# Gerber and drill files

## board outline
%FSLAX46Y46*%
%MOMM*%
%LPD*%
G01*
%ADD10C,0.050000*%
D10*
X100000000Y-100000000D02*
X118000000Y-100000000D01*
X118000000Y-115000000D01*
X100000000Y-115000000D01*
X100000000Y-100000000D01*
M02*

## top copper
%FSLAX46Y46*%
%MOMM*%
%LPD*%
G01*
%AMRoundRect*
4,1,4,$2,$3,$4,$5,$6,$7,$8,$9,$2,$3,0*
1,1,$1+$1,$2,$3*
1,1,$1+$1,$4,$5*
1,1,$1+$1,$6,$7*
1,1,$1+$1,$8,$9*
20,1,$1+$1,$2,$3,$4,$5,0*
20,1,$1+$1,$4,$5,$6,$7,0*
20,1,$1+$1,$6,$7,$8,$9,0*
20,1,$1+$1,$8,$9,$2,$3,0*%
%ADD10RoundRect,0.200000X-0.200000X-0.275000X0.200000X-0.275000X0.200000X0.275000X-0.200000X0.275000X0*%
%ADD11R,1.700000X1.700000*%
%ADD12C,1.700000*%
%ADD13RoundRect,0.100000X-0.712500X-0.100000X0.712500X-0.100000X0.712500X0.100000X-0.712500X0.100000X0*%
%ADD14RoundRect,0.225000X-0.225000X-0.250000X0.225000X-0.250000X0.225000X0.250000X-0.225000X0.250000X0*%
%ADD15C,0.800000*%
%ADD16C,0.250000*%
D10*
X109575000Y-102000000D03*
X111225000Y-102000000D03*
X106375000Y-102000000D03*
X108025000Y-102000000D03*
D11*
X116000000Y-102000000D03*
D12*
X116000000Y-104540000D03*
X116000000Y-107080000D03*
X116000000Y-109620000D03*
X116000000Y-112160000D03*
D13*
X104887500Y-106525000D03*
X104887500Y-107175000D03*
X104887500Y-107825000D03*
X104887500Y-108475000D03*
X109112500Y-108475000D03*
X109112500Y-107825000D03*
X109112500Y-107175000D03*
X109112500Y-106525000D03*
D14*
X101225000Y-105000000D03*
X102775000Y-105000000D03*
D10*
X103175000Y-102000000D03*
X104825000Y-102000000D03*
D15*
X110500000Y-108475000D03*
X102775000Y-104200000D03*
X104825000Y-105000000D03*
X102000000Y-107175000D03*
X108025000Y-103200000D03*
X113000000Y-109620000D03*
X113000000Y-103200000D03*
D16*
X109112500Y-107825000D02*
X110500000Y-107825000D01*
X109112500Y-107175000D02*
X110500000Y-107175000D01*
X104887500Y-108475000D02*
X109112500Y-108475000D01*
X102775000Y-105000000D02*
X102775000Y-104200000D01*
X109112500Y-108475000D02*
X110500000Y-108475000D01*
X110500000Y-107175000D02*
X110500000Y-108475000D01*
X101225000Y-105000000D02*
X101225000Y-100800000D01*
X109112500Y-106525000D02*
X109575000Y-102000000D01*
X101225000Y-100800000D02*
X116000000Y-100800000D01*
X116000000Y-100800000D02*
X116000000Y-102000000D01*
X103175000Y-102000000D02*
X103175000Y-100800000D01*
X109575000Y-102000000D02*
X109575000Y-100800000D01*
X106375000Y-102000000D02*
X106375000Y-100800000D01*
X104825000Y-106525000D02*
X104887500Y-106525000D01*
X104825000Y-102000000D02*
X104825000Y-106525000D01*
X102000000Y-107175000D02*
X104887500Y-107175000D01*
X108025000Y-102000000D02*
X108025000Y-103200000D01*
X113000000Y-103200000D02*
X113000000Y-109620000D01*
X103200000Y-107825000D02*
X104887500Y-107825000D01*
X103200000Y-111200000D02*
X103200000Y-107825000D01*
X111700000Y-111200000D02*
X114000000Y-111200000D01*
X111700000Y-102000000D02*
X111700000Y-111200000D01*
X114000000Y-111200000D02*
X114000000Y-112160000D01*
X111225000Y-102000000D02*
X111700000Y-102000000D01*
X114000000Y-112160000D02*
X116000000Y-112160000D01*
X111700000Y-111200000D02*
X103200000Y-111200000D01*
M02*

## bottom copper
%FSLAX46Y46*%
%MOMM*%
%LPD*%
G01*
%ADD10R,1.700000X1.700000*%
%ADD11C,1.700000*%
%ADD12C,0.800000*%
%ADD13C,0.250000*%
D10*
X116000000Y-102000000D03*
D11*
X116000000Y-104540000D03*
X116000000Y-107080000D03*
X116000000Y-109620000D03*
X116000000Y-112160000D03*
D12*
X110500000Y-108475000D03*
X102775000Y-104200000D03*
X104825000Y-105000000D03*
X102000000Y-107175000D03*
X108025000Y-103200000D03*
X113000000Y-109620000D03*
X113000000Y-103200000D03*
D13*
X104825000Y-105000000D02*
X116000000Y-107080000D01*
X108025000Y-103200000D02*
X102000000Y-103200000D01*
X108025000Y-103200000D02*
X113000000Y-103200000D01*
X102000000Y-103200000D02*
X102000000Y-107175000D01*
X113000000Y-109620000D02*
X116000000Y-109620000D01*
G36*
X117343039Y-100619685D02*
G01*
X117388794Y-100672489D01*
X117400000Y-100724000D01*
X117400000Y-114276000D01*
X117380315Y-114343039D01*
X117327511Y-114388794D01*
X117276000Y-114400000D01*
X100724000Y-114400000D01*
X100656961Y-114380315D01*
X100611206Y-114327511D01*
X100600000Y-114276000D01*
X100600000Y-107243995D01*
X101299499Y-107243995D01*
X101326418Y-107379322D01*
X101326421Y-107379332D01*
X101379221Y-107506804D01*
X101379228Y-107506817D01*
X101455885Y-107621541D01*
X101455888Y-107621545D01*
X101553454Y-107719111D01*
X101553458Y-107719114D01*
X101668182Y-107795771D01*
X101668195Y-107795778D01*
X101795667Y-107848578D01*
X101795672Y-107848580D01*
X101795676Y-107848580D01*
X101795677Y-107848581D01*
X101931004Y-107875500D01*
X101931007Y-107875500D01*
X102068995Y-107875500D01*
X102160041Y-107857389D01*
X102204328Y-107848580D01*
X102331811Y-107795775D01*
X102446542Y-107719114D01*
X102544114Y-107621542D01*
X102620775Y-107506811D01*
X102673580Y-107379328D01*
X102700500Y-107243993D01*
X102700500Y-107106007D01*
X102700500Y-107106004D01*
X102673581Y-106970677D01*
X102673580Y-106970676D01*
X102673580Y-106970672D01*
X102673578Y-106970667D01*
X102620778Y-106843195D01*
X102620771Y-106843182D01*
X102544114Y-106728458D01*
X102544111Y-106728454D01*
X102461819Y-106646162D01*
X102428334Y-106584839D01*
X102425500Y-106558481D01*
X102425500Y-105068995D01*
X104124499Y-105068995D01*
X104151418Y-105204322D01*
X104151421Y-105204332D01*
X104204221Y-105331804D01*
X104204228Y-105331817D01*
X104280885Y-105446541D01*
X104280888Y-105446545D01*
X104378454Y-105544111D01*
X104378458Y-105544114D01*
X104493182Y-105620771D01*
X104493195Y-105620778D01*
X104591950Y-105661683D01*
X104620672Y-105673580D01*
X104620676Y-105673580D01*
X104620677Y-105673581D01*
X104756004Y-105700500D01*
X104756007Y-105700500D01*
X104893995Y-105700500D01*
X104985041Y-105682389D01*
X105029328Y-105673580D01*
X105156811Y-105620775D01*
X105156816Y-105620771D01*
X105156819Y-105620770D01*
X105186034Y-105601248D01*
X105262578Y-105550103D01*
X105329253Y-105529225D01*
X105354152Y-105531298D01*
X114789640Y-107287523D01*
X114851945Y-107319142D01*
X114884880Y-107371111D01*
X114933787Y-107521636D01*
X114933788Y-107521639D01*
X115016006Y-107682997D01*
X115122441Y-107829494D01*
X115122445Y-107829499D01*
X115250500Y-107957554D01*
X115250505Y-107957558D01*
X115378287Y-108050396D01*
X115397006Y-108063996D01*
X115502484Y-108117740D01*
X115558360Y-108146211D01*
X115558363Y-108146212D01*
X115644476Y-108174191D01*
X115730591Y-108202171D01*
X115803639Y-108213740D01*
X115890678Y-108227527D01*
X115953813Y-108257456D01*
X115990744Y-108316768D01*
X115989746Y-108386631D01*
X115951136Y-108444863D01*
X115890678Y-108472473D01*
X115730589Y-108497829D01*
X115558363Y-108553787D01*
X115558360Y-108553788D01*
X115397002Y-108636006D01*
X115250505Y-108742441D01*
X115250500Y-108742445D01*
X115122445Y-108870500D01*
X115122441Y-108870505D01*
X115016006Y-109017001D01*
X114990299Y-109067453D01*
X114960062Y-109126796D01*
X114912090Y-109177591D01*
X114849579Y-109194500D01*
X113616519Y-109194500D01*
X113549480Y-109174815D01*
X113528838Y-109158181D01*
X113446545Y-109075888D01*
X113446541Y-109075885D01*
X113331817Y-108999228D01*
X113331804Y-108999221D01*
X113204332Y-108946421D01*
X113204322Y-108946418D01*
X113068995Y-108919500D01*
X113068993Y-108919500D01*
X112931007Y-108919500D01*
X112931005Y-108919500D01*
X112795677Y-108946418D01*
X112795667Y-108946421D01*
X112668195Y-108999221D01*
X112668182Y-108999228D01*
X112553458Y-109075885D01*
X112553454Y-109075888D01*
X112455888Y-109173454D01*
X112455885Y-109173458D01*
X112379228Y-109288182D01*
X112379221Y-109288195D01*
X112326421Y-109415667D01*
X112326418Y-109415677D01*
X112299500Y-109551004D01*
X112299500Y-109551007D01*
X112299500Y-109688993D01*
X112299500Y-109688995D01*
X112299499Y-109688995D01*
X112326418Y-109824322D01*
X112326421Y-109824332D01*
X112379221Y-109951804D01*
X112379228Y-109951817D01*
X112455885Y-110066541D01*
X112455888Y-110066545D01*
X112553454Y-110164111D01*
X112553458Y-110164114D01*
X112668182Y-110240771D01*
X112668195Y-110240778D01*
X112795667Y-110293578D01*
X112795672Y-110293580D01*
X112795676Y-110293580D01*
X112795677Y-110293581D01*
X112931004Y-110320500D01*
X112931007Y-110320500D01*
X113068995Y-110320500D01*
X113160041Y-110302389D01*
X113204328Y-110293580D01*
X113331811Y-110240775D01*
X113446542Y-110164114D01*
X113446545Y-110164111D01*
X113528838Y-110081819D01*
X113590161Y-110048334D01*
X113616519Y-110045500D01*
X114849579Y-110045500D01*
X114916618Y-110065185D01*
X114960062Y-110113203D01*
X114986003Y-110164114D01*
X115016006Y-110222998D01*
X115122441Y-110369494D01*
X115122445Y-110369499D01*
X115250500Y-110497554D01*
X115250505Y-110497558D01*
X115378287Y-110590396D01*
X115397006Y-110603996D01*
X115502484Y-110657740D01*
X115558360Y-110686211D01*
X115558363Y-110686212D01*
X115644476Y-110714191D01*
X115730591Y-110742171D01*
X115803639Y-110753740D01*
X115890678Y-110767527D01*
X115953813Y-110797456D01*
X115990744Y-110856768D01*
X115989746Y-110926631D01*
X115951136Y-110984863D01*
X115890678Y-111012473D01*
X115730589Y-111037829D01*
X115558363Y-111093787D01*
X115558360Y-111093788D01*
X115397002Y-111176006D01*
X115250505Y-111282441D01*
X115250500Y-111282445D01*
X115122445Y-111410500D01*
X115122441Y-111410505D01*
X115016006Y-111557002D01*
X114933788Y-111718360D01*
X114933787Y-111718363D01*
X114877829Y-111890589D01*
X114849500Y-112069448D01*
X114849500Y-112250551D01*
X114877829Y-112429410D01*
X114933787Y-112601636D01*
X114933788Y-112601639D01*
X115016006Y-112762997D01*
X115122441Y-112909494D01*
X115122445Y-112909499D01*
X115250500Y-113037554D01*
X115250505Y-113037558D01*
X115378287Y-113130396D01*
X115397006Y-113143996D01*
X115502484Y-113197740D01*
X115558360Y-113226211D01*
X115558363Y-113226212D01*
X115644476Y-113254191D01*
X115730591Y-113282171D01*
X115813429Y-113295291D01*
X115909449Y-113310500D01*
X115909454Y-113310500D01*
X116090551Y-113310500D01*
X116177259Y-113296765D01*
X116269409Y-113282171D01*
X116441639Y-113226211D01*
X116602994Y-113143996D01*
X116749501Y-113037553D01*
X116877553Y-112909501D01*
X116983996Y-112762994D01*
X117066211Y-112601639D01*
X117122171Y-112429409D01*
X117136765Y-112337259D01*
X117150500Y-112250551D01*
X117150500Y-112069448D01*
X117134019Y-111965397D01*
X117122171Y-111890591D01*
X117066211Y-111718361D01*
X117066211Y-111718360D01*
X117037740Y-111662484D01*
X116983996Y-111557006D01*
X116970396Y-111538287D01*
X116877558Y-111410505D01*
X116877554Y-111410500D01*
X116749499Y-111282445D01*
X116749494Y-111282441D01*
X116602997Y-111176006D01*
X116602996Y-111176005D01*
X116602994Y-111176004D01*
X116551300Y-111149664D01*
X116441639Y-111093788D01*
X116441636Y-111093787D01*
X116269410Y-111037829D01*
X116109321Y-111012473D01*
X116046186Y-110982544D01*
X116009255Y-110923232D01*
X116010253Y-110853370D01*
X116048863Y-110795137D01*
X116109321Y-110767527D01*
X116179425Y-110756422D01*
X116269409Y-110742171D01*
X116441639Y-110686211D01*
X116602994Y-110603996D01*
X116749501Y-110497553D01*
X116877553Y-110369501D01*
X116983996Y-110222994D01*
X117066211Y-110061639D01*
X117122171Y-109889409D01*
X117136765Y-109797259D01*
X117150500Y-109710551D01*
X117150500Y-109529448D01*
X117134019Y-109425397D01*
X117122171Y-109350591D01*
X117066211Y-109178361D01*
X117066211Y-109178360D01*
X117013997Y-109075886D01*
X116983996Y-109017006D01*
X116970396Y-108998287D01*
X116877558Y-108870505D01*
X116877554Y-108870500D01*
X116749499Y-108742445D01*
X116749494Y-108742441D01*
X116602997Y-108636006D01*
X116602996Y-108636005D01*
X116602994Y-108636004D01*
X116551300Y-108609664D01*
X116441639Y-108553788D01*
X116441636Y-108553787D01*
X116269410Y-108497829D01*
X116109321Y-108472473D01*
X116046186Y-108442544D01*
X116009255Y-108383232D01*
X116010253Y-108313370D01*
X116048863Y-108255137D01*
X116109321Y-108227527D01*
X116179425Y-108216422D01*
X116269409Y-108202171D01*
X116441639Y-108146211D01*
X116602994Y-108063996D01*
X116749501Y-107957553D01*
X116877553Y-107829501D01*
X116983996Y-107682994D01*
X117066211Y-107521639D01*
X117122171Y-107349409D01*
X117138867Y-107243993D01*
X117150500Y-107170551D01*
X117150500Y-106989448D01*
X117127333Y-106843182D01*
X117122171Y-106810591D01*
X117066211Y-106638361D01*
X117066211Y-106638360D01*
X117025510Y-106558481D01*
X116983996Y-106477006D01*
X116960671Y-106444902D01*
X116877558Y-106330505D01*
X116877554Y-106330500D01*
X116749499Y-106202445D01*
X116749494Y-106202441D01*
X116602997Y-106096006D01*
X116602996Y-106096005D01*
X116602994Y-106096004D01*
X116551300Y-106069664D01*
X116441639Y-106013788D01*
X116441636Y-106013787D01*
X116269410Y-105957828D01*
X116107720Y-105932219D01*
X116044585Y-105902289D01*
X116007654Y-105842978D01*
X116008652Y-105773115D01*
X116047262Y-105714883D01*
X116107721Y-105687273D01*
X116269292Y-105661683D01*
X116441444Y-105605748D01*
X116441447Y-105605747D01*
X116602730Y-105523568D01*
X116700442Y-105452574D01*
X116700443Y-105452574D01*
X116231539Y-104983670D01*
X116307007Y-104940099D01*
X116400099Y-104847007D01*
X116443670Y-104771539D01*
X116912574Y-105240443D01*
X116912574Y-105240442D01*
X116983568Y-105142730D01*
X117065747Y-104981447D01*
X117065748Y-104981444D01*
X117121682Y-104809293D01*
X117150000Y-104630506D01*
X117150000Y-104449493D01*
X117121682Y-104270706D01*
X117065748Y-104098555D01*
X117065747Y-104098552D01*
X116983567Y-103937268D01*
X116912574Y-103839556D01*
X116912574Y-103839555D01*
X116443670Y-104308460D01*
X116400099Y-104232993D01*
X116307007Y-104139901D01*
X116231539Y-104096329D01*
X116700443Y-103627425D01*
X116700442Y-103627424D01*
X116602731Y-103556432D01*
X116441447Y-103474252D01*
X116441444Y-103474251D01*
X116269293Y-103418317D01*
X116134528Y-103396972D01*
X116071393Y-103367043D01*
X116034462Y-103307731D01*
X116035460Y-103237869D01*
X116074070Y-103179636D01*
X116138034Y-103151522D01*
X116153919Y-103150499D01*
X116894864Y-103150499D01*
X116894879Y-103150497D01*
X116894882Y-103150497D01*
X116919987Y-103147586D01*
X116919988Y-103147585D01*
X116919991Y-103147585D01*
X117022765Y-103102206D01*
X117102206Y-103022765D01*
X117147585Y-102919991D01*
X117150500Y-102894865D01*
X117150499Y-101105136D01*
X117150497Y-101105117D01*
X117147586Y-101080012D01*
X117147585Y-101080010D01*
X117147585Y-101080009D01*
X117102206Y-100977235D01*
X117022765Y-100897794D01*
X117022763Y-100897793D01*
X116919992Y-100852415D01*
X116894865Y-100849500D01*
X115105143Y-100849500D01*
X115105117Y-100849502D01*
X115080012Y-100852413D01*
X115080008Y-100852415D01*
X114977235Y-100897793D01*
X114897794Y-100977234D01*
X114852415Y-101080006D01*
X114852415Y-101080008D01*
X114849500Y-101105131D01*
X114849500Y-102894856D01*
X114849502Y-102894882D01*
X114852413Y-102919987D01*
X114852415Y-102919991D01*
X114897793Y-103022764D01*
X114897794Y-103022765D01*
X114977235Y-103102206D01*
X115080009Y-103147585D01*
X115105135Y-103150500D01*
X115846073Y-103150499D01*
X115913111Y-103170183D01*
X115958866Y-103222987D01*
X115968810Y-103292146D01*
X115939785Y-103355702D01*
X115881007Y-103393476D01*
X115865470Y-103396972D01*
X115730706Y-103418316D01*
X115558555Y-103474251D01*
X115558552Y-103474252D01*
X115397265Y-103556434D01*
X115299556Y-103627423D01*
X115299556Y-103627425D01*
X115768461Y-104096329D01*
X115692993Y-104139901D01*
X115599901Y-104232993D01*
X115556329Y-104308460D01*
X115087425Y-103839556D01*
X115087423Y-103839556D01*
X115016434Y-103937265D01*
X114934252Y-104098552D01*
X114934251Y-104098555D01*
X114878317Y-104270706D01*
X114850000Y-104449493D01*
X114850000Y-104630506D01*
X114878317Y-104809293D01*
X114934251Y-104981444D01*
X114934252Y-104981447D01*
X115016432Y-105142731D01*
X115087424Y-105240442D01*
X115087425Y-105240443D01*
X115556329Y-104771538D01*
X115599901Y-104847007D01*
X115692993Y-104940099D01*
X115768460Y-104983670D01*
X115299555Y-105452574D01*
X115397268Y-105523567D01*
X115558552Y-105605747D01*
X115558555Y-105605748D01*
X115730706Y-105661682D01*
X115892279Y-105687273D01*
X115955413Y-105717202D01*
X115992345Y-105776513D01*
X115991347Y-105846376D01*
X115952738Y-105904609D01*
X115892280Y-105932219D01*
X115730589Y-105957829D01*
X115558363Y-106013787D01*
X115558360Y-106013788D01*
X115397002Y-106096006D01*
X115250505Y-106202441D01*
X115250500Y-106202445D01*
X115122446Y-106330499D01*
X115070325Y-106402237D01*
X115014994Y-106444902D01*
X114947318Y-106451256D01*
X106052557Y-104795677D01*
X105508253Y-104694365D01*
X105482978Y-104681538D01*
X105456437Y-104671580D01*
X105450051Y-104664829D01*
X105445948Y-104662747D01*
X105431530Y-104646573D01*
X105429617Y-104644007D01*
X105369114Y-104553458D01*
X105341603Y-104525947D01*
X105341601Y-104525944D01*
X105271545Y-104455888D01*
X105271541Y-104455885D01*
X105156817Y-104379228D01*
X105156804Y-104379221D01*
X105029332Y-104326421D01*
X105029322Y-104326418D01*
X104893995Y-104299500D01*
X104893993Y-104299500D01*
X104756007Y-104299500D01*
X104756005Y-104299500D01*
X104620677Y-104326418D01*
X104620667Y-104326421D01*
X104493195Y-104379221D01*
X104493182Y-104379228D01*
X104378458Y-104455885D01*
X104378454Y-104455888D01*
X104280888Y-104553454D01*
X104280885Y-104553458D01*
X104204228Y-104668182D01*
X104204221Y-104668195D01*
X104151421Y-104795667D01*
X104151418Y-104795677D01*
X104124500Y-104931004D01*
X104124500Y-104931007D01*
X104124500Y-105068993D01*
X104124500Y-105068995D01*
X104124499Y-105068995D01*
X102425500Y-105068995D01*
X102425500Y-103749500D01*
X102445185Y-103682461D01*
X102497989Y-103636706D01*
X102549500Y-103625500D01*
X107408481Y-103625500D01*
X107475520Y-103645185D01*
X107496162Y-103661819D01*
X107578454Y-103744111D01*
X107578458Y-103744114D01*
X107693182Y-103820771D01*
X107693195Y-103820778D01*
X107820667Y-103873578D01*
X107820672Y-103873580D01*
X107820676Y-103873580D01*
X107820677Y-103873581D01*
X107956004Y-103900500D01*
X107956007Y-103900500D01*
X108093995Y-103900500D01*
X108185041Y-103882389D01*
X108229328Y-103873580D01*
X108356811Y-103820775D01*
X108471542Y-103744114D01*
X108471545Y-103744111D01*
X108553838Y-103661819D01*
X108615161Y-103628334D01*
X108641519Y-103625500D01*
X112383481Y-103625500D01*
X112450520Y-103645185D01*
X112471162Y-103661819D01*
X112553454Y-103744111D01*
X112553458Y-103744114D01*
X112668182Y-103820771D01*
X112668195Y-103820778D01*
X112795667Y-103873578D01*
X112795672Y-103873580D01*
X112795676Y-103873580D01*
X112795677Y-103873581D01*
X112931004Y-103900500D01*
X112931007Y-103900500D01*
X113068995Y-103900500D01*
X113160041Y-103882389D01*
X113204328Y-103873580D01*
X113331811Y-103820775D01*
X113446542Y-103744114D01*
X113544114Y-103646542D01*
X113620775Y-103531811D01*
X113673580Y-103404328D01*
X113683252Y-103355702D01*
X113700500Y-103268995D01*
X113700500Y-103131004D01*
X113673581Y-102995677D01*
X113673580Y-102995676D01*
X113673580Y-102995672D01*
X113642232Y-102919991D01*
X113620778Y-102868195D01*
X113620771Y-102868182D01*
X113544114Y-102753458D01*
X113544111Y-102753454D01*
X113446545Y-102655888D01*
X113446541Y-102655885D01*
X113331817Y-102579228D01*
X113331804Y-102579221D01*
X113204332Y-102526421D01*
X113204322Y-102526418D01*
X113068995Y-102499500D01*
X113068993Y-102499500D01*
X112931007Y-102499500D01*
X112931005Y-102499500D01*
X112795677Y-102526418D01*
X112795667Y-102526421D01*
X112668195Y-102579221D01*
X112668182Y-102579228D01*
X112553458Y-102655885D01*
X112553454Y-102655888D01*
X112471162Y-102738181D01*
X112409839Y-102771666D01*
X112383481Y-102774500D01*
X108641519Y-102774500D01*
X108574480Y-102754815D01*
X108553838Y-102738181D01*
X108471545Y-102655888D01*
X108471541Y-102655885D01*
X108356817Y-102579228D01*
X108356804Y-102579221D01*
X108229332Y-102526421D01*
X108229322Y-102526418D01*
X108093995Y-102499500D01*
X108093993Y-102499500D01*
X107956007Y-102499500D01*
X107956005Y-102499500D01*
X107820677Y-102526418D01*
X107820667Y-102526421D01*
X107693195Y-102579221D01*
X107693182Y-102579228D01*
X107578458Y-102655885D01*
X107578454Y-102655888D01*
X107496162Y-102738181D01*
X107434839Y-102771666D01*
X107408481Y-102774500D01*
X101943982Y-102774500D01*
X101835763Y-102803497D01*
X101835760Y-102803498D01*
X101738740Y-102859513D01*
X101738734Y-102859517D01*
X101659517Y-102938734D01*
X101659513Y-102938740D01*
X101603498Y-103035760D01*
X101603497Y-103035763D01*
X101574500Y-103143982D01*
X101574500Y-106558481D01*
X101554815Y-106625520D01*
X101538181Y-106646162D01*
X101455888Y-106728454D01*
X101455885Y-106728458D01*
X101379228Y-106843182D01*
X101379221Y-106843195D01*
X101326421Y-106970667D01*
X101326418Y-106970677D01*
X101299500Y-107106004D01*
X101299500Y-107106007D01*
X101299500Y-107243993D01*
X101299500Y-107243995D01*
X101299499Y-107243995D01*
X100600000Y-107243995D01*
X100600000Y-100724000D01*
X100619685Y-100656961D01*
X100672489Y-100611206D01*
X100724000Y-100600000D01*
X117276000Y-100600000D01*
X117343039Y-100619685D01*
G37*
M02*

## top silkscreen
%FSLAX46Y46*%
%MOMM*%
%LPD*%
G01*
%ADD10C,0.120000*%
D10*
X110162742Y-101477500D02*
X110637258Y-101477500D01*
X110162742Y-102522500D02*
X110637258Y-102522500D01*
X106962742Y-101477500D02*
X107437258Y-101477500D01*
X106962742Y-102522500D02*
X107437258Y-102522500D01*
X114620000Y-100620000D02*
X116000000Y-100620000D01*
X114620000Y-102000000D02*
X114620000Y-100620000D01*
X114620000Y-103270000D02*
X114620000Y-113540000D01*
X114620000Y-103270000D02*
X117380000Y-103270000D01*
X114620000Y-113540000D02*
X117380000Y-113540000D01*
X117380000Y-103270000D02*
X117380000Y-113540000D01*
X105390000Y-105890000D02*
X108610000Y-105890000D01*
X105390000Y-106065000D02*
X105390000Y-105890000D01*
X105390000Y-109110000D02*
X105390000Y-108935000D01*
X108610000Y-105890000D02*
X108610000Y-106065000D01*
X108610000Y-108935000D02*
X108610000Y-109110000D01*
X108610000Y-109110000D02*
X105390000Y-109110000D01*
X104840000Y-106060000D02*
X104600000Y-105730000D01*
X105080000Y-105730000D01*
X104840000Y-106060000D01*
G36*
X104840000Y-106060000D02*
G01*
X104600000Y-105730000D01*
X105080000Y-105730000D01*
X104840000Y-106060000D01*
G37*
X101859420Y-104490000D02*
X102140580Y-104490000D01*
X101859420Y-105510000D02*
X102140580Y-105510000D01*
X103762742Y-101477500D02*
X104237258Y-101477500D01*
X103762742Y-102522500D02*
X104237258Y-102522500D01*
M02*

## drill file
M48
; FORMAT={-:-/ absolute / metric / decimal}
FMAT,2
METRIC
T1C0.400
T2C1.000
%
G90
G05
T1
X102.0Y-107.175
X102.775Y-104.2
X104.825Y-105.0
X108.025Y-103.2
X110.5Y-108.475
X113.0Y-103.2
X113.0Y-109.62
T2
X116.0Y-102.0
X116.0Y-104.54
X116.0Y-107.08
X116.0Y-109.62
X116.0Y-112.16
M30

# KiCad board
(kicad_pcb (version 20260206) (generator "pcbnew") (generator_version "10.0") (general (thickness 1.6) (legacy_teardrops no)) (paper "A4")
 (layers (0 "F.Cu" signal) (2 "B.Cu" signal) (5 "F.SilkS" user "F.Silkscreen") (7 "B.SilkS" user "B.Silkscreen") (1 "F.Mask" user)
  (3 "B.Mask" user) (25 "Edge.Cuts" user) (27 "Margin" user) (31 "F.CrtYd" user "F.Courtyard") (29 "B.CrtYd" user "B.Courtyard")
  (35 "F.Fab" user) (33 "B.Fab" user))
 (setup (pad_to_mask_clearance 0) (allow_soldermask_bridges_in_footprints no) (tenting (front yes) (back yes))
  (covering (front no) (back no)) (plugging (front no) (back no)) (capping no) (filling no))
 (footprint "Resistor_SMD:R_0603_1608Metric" (layer "F.Cu") (at 110.4 102)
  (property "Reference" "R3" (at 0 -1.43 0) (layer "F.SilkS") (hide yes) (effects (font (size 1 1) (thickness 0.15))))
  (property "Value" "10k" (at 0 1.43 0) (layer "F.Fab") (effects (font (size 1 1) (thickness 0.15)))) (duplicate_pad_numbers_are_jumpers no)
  (fp_line (start -0.237258 -0.5225) (end 0.237258 -0.5225) (stroke (width 0.12) (type solid)) (layer "F.SilkS"))
  (fp_line (start -0.237258 0.5225) (end 0.237258 0.5225) (stroke (width 0.12) (type solid)) (layer "F.SilkS"))
  (pad "1" smd roundrect (at -0.825 0) (size 0.8 0.95) (layers "F.Cu" "F.Mask" "F.Paste") (roundrect_rratio 0.25) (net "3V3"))
  (pad "2" smd roundrect (at 0.825 0) (size 0.8 0.95) (layers "F.Cu" "F.Mask" "F.Paste") (roundrect_rratio 0.25) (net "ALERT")))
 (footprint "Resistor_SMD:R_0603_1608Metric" (layer "F.Cu") (at 107.2 102)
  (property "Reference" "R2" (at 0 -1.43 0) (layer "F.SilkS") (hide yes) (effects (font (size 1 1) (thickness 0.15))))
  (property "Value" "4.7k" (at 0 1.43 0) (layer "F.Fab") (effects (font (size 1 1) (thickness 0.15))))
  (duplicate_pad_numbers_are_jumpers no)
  (fp_line (start -0.237258 -0.5225) (end 0.237258 -0.5225) (stroke (width 0.12) (type solid)) (layer "F.SilkS"))
  (fp_line (start -0.237258 0.5225) (end 0.237258 0.5225) (stroke (width 0.12) (type solid)) (layer "F.SilkS"))
  (pad "1" smd roundrect (at -0.825 0) (size 0.8 0.95) (layers "F.Cu" "F.Mask" "F.Paste") (roundrect_rratio 0.25) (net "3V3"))
  (pad "2" smd roundrect (at 0.825 0) (size 0.8 0.95) (layers "F.Cu" "F.Mask" "F.Paste") (roundrect_rratio 0.25) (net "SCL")))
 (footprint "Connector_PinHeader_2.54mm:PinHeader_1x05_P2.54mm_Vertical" (layer "F.Cu") (at 116 102)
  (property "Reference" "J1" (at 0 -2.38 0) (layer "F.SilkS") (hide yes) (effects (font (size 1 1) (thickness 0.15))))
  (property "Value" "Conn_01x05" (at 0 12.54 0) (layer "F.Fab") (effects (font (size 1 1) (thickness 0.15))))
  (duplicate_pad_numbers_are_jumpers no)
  (fp_line (start -1.38 -1.38) (end 0 -1.38) (stroke (width 0.12) (type solid)) (layer "F.SilkS"))
  (fp_line (start -1.38 0) (end -1.38 -1.38) (stroke (width 0.12) (type solid)) (layer "F.SilkS"))
  (fp_line (start -1.38 1.27) (end -1.38 11.54) (stroke (width 0.12) (type solid)) (layer "F.SilkS"))
  (fp_line (start -1.38 1.27) (end 1.38 1.27) (stroke (width 0.12) (type solid)) (layer "F.SilkS"))
  (fp_line (start -1.38 11.54) (end 1.38 11.54) (stroke (width 0.12) (type solid)) (layer "F.SilkS"))
  (fp_line (start 1.38 1.27) (end 1.38 11.54) (stroke (width 0.12) (type solid)) (layer "F.SilkS"))
  (pad "1" thru_hole rect (at 0 0) (size 1.7 1.7) (drill 1) (layers "*.Cu" "*.Mask") (remove_unused_layers no) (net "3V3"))
  (pad "2" thru_hole circle (at 0 2.54) (size 1.7 1.7) (drill 1) (layers "*.Cu" "*.Mask") (remove_unused_layers no) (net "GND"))
  (pad "3" thru_hole circle (at 0 5.08) (size 1.7 1.7) (drill 1) (layers "*.Cu" "*.Mask") (remove_unused_layers no) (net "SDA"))
  (pad "4" thru_hole circle (at 0 7.62) (size 1.7 1.7) (drill 1) (layers "*.Cu" "*.Mask") (remove_unused_layers no) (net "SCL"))
  (pad "5" thru_hole circle (at 0 10.16) (size 1.7 1.7) (drill 1) (layers "*.Cu" "*.Mask") (remove_unused_layers no) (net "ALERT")))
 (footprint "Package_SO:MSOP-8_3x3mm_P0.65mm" (layer "F.Cu") (at 107 107.5)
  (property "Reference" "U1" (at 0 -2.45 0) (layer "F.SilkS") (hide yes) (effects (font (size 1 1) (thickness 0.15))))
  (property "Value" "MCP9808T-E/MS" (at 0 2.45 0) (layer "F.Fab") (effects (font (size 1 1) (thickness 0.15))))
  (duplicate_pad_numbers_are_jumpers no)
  (fp_line (start -1.61 -1.61) (end 1.61 -1.61) (stroke (width 0.12) (type solid)) (layer "F.SilkS"))
  (fp_line (start -1.61 -1.435) (end -1.61 -1.61) (stroke (width 0.12) (type solid)) (layer "F.SilkS"))
  (fp_line (start -1.61 1.61) (end -1.61 1.435) (stroke (width 0.12) (type solid)) (layer "F.SilkS"))
  (fp_line (start 1.61 -1.61) (end 1.61 -1.435) (stroke (width 0.12) (type solid)) (layer "F.SilkS"))
  (fp_line (start 1.61 1.435) (end 1.61 1.61) (stroke (width 0.12) (type solid)) (layer "F.SilkS"))
  (fp_line (start 1.61 1.61) (end -1.61 1.61) (stroke (width 0.12) (type solid)) (layer "F.SilkS"))
  (fp_poly (pts (xy -2.16 -1.44) (xy -2.4 -1.77) (xy -1.92 -1.77)) (stroke (width 0.12) (type solid)) (fill yes) (layer "F.SilkS"))
  (pad "1" smd roundrect (at -2.1125 -0.975) (size 1.625 0.4) (layers "F.Cu" "F.Mask" "F.Paste") (roundrect_rratio 0.25) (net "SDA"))
  (pad "2" smd roundrect (at -2.1125 -0.325) (size 1.625 0.4) (layers "F.Cu" "F.Mask" "F.Paste") (roundrect_rratio 0.25) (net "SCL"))
  (pad "3" smd roundrect (at -2.1125 0.325) (size 1.625 0.4) (layers "F.Cu" "F.Mask" "F.Paste") (roundrect_rratio 0.25) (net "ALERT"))
  (pad "4" smd roundrect (at -2.1125 0.975) (size 1.625 0.4) (layers "F.Cu" "F.Mask" "F.Paste") (roundrect_rratio 0.25) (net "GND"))
  (pad "5" smd roundrect (at 2.1125 0.975) (size 1.625 0.4) (layers "F.Cu" "F.Mask" "F.Paste") (roundrect_rratio 0.25) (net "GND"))
  (pad "6" smd roundrect (at 2.1125 0.325) (size 1.625 0.4) (layers "F.Cu" "F.Mask" "F.Paste") (roundrect_rratio 0.25) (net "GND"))
  (pad "7" smd roundrect (at 2.1125 -0.325) (size 1.625 0.4) (layers "F.Cu" "F.Mask" "F.Paste") (roundrect_rratio 0.25) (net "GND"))
  (pad "8" smd roundrect (at 2.1125 -0.975) (size 1.625 0.4) (layers "F.Cu" "F.Mask" "F.Paste") (roundrect_rratio 0.25) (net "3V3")))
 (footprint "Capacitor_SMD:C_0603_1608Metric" (layer "F.Cu") (at 102 105)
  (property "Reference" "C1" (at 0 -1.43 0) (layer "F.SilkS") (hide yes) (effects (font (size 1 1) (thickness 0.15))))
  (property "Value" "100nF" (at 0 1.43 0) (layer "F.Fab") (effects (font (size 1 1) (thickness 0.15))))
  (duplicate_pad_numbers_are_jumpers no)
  (fp_line (start -0.14058 -0.51) (end 0.14058 -0.51) (stroke (width 0.12) (type solid)) (layer "F.SilkS"))
  (fp_line (start -0.14058 0.51) (end 0.14058 0.51) (stroke (width 0.12) (type solid)) (layer "F.SilkS"))
  (pad "1" smd roundrect (at -0.775 0) (size 0.9 0.95) (layers "F.Cu" "F.Mask" "F.Paste") (roundrect_rratio 0.25) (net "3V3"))
  (pad "2" smd roundrect (at 0.775 0) (size 0.9 0.95) (layers "F.Cu" "F.Mask" "F.Paste") (roundrect_rratio 0.25) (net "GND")))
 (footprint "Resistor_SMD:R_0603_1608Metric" (layer "F.Cu") (at 104 102)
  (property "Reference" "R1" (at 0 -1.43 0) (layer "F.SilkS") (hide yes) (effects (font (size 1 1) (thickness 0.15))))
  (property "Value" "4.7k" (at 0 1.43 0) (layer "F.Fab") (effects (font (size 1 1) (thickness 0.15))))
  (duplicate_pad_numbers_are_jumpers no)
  (fp_line (start -0.237258 -0.5225) (end 0.237258 -0.5225) (stroke (width 0.12) (type solid)) (layer "F.SilkS"))
  (fp_line (start -0.237258 0.5225) (end 0.237258 0.5225) (stroke (width 0.12) (type solid)) (layer "F.SilkS"))
  (pad "1" smd roundrect (at -0.825 0) (size 0.8 0.95) (layers "F.Cu" "F.Mask" "F.Paste") (roundrect_rratio 0.25) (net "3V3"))
  (pad "2" smd roundrect (at 0.825 0) (size 0.8 0.95) (layers "F.Cu" "F.Mask" "F.Paste") (roundrect_rratio 0.25) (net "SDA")))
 (gr_rect (start 100 100) (end 118 115) (stroke (width 0.05) (type default)) (fill no) (layer "Edge.Cuts"))
 (segment (start 109.1125 107.825) (end 110.5 107.825) (width 0.25) (layer "F.Cu") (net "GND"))
 (segment (start 109.1125 107.175) (end 110.5 107.175) (width 0.25) (layer "F.Cu") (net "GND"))
 (segment (start 104.8875 108.475) (end 109.1125 108.475) (width 0.25) (layer "F.Cu") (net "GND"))
 (segment (start 102.775 105) (end 102.775 104.2) (width 0.25) (layer "F.Cu") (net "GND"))
 (segment (start 109.1125 108.475) (end 110.5 108.475) (width 0.25) (layer "F.Cu") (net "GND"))
 (segment (start 110.5 107.175) (end 110.5 108.475) (width 0.25) (layer "F.Cu") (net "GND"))
 (via (at 110.5 108.475) (size 0.8) (drill 0.4) (layers "F.Cu" "B.Cu") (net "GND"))
 (via (at 102.775 104.2) (size 0.8) (drill 0.4) (layers "F.Cu" "B.Cu") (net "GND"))
 (segment (start 101.225 105) (end 101.225 100.8) (width 0.25) (layer "F.Cu") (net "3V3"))
 (segment (start 109.1125 106.525) (end 109.575 102) (width 0.25) (layer "F.Cu") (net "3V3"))
 (segment (start 101.225 100.8) (end 116 100.8) (width 0.25) (layer "F.Cu") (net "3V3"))
 (segment (start 116 100.8) (end 116 102) (width 0.25) (layer "F.Cu") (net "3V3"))
 (segment (start 103.175 102) (end 103.175 100.8) (width 0.25) (layer "F.Cu") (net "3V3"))
 (segment (start 109.575 102) (end 109.575 100.8) (width 0.25) (layer "F.Cu") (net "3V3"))
 (segment (start 106.375 102) (end 106.375 100.8) (width 0.25) (layer "F.Cu") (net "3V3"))
 (segment (start 104.825 106.525) (end 104.8875 106.525) (width 0.25) (layer "F.Cu") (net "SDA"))
 (segment (start 104.825 102) (end 104.825 106.525) (width 0.25) (layer "F.Cu") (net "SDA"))
 (via (at 104.825 105) (size 0.8) (drill 0.4) (layers "F.Cu" "B.Cu") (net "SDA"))
 (segment (start 104.825 105) (end 116 107.08) (width 0.25) (layer "B.Cu") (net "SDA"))
 (segment (start 102 107.175) (end 104.8875 107.175) (width 0.25) (layer "F.Cu") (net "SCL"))
 (segment (start 108.025 102) (end 108.025 103.2) (width 0.25) (layer "F.Cu") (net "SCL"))
 (segment (start 113 103.2) (end 113 109.62) (width 0.25) (layer "F.Cu") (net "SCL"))
 (via (at 102 107.175) (size 0.8) (drill 0.4) (layers "F.Cu" "B.Cu") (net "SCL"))
 (via (at 108.025 103.2) (size 0.8) (drill 0.4) (layers "F.Cu" "B.Cu") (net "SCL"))
 (via (at 113 109.62) (size 0.8) (drill 0.4) (layers "F.Cu" "B.Cu") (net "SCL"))
 (via (at 113 103.2) (size 0.8) (drill 0.4) (layers "F.Cu" "B.Cu") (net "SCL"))
 (segment (start 108.025 103.2) (end 102 103.2) (width 0.25) (layer "B.Cu") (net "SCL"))
 (segment (start 108.025 103.2) (end 113 103.2) (width 0.25) (layer "B.Cu") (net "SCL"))
 (segment (start 102 103.2) (end 102 107.175) (width 0.25) (layer "B.Cu") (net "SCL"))
 (segment (start 113 109.62) (end 116 109.62) (width 0.25) (layer "B.Cu") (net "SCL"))
 (segment (start 103.2 107.825) (end 104.8875 107.825) (width 0.25) (layer "F.Cu") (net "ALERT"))
 (segment (start 103.2 111.2) (end 103.2 107.825) (width 0.25) (layer "F.Cu") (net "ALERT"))
 (segment (start 111.7 111.2) (end 114 111.2) (width 0.25) (layer "F.Cu") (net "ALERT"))
 (segment (start 111.7 102) (end 111.7 111.2) (width 0.25) (layer "F.Cu") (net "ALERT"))
 (segment (start 114 111.2) (end 114 112.16) (width 0.25) (layer "F.Cu") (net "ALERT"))
 (segment (start 111.225 102) (end 111.7 102) (width 0.25) (layer "F.Cu") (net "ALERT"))
 (segment (start 114 112.16) (end 116 112.16) (width 0.25) (layer "F.Cu") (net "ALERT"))
 (segment (start 111.7 111.2) (end 103.2 111.2) (width 0.25) (layer "F.Cu") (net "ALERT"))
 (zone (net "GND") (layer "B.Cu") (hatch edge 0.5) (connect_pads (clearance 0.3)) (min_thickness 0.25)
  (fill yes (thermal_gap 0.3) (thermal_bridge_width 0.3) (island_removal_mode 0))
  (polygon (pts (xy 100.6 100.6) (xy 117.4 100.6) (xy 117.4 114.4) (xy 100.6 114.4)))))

